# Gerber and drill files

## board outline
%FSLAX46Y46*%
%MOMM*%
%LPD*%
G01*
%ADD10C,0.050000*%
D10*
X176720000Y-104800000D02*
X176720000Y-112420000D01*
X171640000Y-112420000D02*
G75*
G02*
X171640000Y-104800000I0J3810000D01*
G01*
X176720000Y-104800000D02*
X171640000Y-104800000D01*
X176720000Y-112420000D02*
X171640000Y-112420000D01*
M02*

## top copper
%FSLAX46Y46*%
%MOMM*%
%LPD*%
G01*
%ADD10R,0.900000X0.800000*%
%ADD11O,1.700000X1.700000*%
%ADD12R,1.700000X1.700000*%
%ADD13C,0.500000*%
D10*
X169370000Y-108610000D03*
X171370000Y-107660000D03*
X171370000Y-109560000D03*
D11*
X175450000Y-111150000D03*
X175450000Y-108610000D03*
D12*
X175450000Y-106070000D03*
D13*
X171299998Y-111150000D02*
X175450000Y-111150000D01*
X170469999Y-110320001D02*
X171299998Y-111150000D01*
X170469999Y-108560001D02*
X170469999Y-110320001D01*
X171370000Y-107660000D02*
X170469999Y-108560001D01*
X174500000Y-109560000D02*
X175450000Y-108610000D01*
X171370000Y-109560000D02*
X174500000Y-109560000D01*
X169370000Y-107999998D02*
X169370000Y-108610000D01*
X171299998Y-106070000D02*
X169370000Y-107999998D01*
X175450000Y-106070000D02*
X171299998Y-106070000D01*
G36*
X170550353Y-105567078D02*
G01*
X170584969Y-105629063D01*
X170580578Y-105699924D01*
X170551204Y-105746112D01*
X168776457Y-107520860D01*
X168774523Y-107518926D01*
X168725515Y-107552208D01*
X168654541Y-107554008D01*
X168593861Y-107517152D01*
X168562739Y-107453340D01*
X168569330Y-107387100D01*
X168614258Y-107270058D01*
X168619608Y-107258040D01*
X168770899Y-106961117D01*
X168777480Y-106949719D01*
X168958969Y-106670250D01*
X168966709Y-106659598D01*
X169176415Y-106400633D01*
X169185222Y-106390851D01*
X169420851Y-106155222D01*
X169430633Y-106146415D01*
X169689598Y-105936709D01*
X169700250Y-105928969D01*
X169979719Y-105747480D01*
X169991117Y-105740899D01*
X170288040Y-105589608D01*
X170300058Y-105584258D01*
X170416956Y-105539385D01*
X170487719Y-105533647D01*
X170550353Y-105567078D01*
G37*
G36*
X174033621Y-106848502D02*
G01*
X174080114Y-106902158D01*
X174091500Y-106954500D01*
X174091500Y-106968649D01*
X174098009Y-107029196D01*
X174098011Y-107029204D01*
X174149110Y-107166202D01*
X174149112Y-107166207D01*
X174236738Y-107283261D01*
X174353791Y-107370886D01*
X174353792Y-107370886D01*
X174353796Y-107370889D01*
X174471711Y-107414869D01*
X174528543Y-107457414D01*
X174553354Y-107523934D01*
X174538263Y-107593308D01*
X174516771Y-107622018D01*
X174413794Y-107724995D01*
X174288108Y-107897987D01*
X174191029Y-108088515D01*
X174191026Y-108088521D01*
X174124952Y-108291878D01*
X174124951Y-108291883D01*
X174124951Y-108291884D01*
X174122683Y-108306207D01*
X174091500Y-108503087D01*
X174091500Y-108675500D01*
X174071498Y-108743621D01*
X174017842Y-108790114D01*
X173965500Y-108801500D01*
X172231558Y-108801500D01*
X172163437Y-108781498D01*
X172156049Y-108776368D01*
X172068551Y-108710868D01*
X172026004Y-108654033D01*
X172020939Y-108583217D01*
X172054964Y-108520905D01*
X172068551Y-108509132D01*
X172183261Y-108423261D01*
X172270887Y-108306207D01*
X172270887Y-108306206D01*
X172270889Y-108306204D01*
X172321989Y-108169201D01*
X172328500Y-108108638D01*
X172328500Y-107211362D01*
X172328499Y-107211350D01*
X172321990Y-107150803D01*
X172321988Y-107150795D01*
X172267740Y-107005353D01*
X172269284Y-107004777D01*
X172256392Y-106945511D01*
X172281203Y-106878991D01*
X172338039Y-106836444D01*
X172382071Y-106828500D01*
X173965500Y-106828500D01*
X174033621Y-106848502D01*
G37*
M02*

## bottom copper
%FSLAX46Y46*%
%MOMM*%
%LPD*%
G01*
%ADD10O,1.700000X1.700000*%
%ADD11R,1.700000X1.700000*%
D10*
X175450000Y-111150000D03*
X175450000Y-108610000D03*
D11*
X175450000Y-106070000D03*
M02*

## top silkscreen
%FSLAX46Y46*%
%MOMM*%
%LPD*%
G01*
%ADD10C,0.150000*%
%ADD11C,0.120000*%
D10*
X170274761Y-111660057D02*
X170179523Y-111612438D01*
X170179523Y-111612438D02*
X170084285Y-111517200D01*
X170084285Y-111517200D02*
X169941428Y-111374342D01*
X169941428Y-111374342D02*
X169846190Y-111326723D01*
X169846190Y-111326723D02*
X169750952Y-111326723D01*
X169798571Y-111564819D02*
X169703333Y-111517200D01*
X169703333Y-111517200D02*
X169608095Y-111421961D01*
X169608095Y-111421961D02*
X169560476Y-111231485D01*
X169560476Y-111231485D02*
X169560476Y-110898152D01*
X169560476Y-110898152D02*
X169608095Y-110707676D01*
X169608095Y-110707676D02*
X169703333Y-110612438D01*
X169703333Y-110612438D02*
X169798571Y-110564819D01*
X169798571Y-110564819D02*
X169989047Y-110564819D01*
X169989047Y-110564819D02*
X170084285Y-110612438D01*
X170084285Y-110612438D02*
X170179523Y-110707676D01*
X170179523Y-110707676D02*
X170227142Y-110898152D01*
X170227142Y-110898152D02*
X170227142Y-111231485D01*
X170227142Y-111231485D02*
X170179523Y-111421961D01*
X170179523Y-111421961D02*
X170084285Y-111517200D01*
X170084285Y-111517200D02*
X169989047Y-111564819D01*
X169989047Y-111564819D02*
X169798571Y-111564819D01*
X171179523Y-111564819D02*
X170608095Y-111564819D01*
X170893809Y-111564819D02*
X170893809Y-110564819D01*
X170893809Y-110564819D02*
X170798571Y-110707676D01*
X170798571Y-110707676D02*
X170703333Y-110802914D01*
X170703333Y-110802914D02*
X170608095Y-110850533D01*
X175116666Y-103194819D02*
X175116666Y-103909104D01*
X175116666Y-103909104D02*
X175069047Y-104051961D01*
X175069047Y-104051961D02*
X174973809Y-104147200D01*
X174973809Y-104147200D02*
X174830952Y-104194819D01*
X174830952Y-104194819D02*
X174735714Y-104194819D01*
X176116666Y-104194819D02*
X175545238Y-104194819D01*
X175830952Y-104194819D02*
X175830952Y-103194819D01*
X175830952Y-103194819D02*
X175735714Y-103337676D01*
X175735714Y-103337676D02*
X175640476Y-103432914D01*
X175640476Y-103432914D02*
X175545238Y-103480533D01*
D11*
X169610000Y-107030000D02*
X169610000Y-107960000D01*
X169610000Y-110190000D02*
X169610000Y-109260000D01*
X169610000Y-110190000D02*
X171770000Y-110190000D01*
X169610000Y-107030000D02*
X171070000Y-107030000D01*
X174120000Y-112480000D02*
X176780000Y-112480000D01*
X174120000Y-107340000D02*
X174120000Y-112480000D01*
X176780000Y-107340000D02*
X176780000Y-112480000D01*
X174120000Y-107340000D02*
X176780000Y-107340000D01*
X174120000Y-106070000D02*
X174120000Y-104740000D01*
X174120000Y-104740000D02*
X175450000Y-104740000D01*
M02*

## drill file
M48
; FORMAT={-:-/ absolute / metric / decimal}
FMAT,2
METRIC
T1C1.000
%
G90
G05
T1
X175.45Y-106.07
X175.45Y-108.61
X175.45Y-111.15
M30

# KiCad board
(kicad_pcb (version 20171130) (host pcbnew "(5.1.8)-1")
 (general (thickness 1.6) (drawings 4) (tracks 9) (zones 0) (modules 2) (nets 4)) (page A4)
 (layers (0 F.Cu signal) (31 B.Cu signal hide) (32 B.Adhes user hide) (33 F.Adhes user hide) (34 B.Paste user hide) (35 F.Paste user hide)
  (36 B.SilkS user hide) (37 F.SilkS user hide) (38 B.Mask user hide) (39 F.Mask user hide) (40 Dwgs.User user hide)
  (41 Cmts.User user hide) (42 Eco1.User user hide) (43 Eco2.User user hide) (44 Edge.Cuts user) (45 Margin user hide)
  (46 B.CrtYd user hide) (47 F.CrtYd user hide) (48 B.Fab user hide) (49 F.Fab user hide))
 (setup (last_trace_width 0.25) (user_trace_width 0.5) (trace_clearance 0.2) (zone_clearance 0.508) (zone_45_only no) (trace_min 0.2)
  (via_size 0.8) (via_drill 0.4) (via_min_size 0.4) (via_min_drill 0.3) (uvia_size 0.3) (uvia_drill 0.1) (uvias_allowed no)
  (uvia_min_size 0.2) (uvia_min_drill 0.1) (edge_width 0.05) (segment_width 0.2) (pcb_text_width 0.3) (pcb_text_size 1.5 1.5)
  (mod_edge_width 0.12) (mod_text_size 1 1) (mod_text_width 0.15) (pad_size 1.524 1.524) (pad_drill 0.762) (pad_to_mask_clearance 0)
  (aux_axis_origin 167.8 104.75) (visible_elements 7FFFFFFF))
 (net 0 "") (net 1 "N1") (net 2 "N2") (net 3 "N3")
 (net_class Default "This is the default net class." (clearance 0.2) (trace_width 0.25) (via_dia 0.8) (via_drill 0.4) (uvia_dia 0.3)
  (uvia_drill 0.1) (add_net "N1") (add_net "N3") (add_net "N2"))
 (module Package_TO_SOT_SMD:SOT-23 (layer F.Cu) (at 170.37 108.61 180)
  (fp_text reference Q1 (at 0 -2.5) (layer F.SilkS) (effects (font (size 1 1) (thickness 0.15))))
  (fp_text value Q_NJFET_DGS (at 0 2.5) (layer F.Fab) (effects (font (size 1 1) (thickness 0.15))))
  (fp_line (start 0.76 1.58) (end 0.76 0.65) (layer F.SilkS) (width 0.12))
  (fp_line (start 0.76 -1.58) (end 0.76 -0.65) (layer F.SilkS) (width 0.12))
  (fp_line (start 0.76 -1.58) (end -1.4 -1.58) (layer F.SilkS) (width 0.12))
  (fp_line (start 0.76 1.58) (end -0.7 1.58) (layer F.SilkS) (width 0.12))
  (pad 3 smd rect (at 1 0 180) (size 0.9 0.8) (layers F.Cu F.Paste F.Mask) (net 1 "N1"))
  (pad 2 smd rect (at -1 0.95 180) (size 0.9 0.8) (layers F.Cu F.Paste F.Mask) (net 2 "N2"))
  (pad 1 smd rect (at -1 -0.95 180) (size 0.9 0.8) (layers F.Cu F.Paste F.Mask) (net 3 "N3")))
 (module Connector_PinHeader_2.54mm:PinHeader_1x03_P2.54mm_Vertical (layer F.Cu) (at 175.45 106.07)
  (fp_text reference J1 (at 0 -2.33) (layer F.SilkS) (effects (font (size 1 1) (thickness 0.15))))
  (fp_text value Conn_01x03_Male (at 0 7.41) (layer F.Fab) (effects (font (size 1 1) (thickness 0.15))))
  (fp_line (start -1.33 6.41) (end 1.33 6.41) (layer F.SilkS) (width 0.12))
  (fp_line (start -1.33 1.27) (end -1.33 6.41) (layer F.SilkS) (width 0.12))
  (fp_line (start 1.33 1.27) (end 1.33 6.41) (layer F.SilkS) (width 0.12))
  (fp_line (start -1.33 1.27) (end 1.33 1.27) (layer F.SilkS) (width 0.12))
  (fp_line (start -1.33 0) (end -1.33 -1.33) (layer F.SilkS) (width 0.12))
  (fp_line (start -1.33 -1.33) (end 0 -1.33) (layer F.SilkS) (width 0.12))
  (pad 3 thru_hole oval (at 0 5.08) (size 1.7 1.7) (drill 1) (layers *.Cu *.Mask) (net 2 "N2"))
  (pad 2 thru_hole oval (at 0 2.54) (size 1.7 1.7) (drill 1) (layers *.Cu *.Mask) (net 3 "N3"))
  (pad 1 thru_hole rect (at 0 0) (size 1.7 1.7) (drill 1) (layers *.Cu *.Mask) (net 1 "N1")))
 (gr_line (start 176.72 104.8) (end 176.72 112.42) (layer Edge.Cuts) (width 0.05))
 (gr_arc (start 171.64 108.61) (end 171.64 104.8) (angle -180) (layer Edge.Cuts) (width 0.05))
 (gr_line (start 176.72 104.8) (end 171.64 104.8) (layer Edge.Cuts) (width 0.05))
 (gr_line (start 176.72 112.42) (end 171.64 112.42) (layer Edge.Cuts) (width 0.05))
 (segment (start 171.299998 111.15) (end 175.45 111.15) (width 0.5) (layer F.Cu) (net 2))
 (segment (start 170.469999 110.320001) (end 171.299998 111.15) (width 0.5) (layer F.Cu) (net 2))
 (segment (start 170.469999 108.560001) (end 170.469999 110.320001) (width 0.5) (layer F.Cu) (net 2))
 (segment (start 171.37 107.66) (end 170.469999 108.560001) (width 0.5) (layer F.Cu) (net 2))
 (segment (start 174.5 109.56) (end 175.45 108.61) (width 0.5) (layer F.Cu) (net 3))
 (segment (start 171.37 109.56) (end 174.5 109.56) (width 0.5) (layer F.Cu) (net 3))
 (segment (start 169.37 107.999998) (end 169.37 108.61) (width 0.5) (layer F.Cu) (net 1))
 (segment (start 171.299998 106.07) (end 169.37 107.999998) (width 0.5) (layer F.Cu) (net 1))
 (segment (start 175.45 106.07) (end 171.299998 106.07) (width 0.5) (layer F.Cu) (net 1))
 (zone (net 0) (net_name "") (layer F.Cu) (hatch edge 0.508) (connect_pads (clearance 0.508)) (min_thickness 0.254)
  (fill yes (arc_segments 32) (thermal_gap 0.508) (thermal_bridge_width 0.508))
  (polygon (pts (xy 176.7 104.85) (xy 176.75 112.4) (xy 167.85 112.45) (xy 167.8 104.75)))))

